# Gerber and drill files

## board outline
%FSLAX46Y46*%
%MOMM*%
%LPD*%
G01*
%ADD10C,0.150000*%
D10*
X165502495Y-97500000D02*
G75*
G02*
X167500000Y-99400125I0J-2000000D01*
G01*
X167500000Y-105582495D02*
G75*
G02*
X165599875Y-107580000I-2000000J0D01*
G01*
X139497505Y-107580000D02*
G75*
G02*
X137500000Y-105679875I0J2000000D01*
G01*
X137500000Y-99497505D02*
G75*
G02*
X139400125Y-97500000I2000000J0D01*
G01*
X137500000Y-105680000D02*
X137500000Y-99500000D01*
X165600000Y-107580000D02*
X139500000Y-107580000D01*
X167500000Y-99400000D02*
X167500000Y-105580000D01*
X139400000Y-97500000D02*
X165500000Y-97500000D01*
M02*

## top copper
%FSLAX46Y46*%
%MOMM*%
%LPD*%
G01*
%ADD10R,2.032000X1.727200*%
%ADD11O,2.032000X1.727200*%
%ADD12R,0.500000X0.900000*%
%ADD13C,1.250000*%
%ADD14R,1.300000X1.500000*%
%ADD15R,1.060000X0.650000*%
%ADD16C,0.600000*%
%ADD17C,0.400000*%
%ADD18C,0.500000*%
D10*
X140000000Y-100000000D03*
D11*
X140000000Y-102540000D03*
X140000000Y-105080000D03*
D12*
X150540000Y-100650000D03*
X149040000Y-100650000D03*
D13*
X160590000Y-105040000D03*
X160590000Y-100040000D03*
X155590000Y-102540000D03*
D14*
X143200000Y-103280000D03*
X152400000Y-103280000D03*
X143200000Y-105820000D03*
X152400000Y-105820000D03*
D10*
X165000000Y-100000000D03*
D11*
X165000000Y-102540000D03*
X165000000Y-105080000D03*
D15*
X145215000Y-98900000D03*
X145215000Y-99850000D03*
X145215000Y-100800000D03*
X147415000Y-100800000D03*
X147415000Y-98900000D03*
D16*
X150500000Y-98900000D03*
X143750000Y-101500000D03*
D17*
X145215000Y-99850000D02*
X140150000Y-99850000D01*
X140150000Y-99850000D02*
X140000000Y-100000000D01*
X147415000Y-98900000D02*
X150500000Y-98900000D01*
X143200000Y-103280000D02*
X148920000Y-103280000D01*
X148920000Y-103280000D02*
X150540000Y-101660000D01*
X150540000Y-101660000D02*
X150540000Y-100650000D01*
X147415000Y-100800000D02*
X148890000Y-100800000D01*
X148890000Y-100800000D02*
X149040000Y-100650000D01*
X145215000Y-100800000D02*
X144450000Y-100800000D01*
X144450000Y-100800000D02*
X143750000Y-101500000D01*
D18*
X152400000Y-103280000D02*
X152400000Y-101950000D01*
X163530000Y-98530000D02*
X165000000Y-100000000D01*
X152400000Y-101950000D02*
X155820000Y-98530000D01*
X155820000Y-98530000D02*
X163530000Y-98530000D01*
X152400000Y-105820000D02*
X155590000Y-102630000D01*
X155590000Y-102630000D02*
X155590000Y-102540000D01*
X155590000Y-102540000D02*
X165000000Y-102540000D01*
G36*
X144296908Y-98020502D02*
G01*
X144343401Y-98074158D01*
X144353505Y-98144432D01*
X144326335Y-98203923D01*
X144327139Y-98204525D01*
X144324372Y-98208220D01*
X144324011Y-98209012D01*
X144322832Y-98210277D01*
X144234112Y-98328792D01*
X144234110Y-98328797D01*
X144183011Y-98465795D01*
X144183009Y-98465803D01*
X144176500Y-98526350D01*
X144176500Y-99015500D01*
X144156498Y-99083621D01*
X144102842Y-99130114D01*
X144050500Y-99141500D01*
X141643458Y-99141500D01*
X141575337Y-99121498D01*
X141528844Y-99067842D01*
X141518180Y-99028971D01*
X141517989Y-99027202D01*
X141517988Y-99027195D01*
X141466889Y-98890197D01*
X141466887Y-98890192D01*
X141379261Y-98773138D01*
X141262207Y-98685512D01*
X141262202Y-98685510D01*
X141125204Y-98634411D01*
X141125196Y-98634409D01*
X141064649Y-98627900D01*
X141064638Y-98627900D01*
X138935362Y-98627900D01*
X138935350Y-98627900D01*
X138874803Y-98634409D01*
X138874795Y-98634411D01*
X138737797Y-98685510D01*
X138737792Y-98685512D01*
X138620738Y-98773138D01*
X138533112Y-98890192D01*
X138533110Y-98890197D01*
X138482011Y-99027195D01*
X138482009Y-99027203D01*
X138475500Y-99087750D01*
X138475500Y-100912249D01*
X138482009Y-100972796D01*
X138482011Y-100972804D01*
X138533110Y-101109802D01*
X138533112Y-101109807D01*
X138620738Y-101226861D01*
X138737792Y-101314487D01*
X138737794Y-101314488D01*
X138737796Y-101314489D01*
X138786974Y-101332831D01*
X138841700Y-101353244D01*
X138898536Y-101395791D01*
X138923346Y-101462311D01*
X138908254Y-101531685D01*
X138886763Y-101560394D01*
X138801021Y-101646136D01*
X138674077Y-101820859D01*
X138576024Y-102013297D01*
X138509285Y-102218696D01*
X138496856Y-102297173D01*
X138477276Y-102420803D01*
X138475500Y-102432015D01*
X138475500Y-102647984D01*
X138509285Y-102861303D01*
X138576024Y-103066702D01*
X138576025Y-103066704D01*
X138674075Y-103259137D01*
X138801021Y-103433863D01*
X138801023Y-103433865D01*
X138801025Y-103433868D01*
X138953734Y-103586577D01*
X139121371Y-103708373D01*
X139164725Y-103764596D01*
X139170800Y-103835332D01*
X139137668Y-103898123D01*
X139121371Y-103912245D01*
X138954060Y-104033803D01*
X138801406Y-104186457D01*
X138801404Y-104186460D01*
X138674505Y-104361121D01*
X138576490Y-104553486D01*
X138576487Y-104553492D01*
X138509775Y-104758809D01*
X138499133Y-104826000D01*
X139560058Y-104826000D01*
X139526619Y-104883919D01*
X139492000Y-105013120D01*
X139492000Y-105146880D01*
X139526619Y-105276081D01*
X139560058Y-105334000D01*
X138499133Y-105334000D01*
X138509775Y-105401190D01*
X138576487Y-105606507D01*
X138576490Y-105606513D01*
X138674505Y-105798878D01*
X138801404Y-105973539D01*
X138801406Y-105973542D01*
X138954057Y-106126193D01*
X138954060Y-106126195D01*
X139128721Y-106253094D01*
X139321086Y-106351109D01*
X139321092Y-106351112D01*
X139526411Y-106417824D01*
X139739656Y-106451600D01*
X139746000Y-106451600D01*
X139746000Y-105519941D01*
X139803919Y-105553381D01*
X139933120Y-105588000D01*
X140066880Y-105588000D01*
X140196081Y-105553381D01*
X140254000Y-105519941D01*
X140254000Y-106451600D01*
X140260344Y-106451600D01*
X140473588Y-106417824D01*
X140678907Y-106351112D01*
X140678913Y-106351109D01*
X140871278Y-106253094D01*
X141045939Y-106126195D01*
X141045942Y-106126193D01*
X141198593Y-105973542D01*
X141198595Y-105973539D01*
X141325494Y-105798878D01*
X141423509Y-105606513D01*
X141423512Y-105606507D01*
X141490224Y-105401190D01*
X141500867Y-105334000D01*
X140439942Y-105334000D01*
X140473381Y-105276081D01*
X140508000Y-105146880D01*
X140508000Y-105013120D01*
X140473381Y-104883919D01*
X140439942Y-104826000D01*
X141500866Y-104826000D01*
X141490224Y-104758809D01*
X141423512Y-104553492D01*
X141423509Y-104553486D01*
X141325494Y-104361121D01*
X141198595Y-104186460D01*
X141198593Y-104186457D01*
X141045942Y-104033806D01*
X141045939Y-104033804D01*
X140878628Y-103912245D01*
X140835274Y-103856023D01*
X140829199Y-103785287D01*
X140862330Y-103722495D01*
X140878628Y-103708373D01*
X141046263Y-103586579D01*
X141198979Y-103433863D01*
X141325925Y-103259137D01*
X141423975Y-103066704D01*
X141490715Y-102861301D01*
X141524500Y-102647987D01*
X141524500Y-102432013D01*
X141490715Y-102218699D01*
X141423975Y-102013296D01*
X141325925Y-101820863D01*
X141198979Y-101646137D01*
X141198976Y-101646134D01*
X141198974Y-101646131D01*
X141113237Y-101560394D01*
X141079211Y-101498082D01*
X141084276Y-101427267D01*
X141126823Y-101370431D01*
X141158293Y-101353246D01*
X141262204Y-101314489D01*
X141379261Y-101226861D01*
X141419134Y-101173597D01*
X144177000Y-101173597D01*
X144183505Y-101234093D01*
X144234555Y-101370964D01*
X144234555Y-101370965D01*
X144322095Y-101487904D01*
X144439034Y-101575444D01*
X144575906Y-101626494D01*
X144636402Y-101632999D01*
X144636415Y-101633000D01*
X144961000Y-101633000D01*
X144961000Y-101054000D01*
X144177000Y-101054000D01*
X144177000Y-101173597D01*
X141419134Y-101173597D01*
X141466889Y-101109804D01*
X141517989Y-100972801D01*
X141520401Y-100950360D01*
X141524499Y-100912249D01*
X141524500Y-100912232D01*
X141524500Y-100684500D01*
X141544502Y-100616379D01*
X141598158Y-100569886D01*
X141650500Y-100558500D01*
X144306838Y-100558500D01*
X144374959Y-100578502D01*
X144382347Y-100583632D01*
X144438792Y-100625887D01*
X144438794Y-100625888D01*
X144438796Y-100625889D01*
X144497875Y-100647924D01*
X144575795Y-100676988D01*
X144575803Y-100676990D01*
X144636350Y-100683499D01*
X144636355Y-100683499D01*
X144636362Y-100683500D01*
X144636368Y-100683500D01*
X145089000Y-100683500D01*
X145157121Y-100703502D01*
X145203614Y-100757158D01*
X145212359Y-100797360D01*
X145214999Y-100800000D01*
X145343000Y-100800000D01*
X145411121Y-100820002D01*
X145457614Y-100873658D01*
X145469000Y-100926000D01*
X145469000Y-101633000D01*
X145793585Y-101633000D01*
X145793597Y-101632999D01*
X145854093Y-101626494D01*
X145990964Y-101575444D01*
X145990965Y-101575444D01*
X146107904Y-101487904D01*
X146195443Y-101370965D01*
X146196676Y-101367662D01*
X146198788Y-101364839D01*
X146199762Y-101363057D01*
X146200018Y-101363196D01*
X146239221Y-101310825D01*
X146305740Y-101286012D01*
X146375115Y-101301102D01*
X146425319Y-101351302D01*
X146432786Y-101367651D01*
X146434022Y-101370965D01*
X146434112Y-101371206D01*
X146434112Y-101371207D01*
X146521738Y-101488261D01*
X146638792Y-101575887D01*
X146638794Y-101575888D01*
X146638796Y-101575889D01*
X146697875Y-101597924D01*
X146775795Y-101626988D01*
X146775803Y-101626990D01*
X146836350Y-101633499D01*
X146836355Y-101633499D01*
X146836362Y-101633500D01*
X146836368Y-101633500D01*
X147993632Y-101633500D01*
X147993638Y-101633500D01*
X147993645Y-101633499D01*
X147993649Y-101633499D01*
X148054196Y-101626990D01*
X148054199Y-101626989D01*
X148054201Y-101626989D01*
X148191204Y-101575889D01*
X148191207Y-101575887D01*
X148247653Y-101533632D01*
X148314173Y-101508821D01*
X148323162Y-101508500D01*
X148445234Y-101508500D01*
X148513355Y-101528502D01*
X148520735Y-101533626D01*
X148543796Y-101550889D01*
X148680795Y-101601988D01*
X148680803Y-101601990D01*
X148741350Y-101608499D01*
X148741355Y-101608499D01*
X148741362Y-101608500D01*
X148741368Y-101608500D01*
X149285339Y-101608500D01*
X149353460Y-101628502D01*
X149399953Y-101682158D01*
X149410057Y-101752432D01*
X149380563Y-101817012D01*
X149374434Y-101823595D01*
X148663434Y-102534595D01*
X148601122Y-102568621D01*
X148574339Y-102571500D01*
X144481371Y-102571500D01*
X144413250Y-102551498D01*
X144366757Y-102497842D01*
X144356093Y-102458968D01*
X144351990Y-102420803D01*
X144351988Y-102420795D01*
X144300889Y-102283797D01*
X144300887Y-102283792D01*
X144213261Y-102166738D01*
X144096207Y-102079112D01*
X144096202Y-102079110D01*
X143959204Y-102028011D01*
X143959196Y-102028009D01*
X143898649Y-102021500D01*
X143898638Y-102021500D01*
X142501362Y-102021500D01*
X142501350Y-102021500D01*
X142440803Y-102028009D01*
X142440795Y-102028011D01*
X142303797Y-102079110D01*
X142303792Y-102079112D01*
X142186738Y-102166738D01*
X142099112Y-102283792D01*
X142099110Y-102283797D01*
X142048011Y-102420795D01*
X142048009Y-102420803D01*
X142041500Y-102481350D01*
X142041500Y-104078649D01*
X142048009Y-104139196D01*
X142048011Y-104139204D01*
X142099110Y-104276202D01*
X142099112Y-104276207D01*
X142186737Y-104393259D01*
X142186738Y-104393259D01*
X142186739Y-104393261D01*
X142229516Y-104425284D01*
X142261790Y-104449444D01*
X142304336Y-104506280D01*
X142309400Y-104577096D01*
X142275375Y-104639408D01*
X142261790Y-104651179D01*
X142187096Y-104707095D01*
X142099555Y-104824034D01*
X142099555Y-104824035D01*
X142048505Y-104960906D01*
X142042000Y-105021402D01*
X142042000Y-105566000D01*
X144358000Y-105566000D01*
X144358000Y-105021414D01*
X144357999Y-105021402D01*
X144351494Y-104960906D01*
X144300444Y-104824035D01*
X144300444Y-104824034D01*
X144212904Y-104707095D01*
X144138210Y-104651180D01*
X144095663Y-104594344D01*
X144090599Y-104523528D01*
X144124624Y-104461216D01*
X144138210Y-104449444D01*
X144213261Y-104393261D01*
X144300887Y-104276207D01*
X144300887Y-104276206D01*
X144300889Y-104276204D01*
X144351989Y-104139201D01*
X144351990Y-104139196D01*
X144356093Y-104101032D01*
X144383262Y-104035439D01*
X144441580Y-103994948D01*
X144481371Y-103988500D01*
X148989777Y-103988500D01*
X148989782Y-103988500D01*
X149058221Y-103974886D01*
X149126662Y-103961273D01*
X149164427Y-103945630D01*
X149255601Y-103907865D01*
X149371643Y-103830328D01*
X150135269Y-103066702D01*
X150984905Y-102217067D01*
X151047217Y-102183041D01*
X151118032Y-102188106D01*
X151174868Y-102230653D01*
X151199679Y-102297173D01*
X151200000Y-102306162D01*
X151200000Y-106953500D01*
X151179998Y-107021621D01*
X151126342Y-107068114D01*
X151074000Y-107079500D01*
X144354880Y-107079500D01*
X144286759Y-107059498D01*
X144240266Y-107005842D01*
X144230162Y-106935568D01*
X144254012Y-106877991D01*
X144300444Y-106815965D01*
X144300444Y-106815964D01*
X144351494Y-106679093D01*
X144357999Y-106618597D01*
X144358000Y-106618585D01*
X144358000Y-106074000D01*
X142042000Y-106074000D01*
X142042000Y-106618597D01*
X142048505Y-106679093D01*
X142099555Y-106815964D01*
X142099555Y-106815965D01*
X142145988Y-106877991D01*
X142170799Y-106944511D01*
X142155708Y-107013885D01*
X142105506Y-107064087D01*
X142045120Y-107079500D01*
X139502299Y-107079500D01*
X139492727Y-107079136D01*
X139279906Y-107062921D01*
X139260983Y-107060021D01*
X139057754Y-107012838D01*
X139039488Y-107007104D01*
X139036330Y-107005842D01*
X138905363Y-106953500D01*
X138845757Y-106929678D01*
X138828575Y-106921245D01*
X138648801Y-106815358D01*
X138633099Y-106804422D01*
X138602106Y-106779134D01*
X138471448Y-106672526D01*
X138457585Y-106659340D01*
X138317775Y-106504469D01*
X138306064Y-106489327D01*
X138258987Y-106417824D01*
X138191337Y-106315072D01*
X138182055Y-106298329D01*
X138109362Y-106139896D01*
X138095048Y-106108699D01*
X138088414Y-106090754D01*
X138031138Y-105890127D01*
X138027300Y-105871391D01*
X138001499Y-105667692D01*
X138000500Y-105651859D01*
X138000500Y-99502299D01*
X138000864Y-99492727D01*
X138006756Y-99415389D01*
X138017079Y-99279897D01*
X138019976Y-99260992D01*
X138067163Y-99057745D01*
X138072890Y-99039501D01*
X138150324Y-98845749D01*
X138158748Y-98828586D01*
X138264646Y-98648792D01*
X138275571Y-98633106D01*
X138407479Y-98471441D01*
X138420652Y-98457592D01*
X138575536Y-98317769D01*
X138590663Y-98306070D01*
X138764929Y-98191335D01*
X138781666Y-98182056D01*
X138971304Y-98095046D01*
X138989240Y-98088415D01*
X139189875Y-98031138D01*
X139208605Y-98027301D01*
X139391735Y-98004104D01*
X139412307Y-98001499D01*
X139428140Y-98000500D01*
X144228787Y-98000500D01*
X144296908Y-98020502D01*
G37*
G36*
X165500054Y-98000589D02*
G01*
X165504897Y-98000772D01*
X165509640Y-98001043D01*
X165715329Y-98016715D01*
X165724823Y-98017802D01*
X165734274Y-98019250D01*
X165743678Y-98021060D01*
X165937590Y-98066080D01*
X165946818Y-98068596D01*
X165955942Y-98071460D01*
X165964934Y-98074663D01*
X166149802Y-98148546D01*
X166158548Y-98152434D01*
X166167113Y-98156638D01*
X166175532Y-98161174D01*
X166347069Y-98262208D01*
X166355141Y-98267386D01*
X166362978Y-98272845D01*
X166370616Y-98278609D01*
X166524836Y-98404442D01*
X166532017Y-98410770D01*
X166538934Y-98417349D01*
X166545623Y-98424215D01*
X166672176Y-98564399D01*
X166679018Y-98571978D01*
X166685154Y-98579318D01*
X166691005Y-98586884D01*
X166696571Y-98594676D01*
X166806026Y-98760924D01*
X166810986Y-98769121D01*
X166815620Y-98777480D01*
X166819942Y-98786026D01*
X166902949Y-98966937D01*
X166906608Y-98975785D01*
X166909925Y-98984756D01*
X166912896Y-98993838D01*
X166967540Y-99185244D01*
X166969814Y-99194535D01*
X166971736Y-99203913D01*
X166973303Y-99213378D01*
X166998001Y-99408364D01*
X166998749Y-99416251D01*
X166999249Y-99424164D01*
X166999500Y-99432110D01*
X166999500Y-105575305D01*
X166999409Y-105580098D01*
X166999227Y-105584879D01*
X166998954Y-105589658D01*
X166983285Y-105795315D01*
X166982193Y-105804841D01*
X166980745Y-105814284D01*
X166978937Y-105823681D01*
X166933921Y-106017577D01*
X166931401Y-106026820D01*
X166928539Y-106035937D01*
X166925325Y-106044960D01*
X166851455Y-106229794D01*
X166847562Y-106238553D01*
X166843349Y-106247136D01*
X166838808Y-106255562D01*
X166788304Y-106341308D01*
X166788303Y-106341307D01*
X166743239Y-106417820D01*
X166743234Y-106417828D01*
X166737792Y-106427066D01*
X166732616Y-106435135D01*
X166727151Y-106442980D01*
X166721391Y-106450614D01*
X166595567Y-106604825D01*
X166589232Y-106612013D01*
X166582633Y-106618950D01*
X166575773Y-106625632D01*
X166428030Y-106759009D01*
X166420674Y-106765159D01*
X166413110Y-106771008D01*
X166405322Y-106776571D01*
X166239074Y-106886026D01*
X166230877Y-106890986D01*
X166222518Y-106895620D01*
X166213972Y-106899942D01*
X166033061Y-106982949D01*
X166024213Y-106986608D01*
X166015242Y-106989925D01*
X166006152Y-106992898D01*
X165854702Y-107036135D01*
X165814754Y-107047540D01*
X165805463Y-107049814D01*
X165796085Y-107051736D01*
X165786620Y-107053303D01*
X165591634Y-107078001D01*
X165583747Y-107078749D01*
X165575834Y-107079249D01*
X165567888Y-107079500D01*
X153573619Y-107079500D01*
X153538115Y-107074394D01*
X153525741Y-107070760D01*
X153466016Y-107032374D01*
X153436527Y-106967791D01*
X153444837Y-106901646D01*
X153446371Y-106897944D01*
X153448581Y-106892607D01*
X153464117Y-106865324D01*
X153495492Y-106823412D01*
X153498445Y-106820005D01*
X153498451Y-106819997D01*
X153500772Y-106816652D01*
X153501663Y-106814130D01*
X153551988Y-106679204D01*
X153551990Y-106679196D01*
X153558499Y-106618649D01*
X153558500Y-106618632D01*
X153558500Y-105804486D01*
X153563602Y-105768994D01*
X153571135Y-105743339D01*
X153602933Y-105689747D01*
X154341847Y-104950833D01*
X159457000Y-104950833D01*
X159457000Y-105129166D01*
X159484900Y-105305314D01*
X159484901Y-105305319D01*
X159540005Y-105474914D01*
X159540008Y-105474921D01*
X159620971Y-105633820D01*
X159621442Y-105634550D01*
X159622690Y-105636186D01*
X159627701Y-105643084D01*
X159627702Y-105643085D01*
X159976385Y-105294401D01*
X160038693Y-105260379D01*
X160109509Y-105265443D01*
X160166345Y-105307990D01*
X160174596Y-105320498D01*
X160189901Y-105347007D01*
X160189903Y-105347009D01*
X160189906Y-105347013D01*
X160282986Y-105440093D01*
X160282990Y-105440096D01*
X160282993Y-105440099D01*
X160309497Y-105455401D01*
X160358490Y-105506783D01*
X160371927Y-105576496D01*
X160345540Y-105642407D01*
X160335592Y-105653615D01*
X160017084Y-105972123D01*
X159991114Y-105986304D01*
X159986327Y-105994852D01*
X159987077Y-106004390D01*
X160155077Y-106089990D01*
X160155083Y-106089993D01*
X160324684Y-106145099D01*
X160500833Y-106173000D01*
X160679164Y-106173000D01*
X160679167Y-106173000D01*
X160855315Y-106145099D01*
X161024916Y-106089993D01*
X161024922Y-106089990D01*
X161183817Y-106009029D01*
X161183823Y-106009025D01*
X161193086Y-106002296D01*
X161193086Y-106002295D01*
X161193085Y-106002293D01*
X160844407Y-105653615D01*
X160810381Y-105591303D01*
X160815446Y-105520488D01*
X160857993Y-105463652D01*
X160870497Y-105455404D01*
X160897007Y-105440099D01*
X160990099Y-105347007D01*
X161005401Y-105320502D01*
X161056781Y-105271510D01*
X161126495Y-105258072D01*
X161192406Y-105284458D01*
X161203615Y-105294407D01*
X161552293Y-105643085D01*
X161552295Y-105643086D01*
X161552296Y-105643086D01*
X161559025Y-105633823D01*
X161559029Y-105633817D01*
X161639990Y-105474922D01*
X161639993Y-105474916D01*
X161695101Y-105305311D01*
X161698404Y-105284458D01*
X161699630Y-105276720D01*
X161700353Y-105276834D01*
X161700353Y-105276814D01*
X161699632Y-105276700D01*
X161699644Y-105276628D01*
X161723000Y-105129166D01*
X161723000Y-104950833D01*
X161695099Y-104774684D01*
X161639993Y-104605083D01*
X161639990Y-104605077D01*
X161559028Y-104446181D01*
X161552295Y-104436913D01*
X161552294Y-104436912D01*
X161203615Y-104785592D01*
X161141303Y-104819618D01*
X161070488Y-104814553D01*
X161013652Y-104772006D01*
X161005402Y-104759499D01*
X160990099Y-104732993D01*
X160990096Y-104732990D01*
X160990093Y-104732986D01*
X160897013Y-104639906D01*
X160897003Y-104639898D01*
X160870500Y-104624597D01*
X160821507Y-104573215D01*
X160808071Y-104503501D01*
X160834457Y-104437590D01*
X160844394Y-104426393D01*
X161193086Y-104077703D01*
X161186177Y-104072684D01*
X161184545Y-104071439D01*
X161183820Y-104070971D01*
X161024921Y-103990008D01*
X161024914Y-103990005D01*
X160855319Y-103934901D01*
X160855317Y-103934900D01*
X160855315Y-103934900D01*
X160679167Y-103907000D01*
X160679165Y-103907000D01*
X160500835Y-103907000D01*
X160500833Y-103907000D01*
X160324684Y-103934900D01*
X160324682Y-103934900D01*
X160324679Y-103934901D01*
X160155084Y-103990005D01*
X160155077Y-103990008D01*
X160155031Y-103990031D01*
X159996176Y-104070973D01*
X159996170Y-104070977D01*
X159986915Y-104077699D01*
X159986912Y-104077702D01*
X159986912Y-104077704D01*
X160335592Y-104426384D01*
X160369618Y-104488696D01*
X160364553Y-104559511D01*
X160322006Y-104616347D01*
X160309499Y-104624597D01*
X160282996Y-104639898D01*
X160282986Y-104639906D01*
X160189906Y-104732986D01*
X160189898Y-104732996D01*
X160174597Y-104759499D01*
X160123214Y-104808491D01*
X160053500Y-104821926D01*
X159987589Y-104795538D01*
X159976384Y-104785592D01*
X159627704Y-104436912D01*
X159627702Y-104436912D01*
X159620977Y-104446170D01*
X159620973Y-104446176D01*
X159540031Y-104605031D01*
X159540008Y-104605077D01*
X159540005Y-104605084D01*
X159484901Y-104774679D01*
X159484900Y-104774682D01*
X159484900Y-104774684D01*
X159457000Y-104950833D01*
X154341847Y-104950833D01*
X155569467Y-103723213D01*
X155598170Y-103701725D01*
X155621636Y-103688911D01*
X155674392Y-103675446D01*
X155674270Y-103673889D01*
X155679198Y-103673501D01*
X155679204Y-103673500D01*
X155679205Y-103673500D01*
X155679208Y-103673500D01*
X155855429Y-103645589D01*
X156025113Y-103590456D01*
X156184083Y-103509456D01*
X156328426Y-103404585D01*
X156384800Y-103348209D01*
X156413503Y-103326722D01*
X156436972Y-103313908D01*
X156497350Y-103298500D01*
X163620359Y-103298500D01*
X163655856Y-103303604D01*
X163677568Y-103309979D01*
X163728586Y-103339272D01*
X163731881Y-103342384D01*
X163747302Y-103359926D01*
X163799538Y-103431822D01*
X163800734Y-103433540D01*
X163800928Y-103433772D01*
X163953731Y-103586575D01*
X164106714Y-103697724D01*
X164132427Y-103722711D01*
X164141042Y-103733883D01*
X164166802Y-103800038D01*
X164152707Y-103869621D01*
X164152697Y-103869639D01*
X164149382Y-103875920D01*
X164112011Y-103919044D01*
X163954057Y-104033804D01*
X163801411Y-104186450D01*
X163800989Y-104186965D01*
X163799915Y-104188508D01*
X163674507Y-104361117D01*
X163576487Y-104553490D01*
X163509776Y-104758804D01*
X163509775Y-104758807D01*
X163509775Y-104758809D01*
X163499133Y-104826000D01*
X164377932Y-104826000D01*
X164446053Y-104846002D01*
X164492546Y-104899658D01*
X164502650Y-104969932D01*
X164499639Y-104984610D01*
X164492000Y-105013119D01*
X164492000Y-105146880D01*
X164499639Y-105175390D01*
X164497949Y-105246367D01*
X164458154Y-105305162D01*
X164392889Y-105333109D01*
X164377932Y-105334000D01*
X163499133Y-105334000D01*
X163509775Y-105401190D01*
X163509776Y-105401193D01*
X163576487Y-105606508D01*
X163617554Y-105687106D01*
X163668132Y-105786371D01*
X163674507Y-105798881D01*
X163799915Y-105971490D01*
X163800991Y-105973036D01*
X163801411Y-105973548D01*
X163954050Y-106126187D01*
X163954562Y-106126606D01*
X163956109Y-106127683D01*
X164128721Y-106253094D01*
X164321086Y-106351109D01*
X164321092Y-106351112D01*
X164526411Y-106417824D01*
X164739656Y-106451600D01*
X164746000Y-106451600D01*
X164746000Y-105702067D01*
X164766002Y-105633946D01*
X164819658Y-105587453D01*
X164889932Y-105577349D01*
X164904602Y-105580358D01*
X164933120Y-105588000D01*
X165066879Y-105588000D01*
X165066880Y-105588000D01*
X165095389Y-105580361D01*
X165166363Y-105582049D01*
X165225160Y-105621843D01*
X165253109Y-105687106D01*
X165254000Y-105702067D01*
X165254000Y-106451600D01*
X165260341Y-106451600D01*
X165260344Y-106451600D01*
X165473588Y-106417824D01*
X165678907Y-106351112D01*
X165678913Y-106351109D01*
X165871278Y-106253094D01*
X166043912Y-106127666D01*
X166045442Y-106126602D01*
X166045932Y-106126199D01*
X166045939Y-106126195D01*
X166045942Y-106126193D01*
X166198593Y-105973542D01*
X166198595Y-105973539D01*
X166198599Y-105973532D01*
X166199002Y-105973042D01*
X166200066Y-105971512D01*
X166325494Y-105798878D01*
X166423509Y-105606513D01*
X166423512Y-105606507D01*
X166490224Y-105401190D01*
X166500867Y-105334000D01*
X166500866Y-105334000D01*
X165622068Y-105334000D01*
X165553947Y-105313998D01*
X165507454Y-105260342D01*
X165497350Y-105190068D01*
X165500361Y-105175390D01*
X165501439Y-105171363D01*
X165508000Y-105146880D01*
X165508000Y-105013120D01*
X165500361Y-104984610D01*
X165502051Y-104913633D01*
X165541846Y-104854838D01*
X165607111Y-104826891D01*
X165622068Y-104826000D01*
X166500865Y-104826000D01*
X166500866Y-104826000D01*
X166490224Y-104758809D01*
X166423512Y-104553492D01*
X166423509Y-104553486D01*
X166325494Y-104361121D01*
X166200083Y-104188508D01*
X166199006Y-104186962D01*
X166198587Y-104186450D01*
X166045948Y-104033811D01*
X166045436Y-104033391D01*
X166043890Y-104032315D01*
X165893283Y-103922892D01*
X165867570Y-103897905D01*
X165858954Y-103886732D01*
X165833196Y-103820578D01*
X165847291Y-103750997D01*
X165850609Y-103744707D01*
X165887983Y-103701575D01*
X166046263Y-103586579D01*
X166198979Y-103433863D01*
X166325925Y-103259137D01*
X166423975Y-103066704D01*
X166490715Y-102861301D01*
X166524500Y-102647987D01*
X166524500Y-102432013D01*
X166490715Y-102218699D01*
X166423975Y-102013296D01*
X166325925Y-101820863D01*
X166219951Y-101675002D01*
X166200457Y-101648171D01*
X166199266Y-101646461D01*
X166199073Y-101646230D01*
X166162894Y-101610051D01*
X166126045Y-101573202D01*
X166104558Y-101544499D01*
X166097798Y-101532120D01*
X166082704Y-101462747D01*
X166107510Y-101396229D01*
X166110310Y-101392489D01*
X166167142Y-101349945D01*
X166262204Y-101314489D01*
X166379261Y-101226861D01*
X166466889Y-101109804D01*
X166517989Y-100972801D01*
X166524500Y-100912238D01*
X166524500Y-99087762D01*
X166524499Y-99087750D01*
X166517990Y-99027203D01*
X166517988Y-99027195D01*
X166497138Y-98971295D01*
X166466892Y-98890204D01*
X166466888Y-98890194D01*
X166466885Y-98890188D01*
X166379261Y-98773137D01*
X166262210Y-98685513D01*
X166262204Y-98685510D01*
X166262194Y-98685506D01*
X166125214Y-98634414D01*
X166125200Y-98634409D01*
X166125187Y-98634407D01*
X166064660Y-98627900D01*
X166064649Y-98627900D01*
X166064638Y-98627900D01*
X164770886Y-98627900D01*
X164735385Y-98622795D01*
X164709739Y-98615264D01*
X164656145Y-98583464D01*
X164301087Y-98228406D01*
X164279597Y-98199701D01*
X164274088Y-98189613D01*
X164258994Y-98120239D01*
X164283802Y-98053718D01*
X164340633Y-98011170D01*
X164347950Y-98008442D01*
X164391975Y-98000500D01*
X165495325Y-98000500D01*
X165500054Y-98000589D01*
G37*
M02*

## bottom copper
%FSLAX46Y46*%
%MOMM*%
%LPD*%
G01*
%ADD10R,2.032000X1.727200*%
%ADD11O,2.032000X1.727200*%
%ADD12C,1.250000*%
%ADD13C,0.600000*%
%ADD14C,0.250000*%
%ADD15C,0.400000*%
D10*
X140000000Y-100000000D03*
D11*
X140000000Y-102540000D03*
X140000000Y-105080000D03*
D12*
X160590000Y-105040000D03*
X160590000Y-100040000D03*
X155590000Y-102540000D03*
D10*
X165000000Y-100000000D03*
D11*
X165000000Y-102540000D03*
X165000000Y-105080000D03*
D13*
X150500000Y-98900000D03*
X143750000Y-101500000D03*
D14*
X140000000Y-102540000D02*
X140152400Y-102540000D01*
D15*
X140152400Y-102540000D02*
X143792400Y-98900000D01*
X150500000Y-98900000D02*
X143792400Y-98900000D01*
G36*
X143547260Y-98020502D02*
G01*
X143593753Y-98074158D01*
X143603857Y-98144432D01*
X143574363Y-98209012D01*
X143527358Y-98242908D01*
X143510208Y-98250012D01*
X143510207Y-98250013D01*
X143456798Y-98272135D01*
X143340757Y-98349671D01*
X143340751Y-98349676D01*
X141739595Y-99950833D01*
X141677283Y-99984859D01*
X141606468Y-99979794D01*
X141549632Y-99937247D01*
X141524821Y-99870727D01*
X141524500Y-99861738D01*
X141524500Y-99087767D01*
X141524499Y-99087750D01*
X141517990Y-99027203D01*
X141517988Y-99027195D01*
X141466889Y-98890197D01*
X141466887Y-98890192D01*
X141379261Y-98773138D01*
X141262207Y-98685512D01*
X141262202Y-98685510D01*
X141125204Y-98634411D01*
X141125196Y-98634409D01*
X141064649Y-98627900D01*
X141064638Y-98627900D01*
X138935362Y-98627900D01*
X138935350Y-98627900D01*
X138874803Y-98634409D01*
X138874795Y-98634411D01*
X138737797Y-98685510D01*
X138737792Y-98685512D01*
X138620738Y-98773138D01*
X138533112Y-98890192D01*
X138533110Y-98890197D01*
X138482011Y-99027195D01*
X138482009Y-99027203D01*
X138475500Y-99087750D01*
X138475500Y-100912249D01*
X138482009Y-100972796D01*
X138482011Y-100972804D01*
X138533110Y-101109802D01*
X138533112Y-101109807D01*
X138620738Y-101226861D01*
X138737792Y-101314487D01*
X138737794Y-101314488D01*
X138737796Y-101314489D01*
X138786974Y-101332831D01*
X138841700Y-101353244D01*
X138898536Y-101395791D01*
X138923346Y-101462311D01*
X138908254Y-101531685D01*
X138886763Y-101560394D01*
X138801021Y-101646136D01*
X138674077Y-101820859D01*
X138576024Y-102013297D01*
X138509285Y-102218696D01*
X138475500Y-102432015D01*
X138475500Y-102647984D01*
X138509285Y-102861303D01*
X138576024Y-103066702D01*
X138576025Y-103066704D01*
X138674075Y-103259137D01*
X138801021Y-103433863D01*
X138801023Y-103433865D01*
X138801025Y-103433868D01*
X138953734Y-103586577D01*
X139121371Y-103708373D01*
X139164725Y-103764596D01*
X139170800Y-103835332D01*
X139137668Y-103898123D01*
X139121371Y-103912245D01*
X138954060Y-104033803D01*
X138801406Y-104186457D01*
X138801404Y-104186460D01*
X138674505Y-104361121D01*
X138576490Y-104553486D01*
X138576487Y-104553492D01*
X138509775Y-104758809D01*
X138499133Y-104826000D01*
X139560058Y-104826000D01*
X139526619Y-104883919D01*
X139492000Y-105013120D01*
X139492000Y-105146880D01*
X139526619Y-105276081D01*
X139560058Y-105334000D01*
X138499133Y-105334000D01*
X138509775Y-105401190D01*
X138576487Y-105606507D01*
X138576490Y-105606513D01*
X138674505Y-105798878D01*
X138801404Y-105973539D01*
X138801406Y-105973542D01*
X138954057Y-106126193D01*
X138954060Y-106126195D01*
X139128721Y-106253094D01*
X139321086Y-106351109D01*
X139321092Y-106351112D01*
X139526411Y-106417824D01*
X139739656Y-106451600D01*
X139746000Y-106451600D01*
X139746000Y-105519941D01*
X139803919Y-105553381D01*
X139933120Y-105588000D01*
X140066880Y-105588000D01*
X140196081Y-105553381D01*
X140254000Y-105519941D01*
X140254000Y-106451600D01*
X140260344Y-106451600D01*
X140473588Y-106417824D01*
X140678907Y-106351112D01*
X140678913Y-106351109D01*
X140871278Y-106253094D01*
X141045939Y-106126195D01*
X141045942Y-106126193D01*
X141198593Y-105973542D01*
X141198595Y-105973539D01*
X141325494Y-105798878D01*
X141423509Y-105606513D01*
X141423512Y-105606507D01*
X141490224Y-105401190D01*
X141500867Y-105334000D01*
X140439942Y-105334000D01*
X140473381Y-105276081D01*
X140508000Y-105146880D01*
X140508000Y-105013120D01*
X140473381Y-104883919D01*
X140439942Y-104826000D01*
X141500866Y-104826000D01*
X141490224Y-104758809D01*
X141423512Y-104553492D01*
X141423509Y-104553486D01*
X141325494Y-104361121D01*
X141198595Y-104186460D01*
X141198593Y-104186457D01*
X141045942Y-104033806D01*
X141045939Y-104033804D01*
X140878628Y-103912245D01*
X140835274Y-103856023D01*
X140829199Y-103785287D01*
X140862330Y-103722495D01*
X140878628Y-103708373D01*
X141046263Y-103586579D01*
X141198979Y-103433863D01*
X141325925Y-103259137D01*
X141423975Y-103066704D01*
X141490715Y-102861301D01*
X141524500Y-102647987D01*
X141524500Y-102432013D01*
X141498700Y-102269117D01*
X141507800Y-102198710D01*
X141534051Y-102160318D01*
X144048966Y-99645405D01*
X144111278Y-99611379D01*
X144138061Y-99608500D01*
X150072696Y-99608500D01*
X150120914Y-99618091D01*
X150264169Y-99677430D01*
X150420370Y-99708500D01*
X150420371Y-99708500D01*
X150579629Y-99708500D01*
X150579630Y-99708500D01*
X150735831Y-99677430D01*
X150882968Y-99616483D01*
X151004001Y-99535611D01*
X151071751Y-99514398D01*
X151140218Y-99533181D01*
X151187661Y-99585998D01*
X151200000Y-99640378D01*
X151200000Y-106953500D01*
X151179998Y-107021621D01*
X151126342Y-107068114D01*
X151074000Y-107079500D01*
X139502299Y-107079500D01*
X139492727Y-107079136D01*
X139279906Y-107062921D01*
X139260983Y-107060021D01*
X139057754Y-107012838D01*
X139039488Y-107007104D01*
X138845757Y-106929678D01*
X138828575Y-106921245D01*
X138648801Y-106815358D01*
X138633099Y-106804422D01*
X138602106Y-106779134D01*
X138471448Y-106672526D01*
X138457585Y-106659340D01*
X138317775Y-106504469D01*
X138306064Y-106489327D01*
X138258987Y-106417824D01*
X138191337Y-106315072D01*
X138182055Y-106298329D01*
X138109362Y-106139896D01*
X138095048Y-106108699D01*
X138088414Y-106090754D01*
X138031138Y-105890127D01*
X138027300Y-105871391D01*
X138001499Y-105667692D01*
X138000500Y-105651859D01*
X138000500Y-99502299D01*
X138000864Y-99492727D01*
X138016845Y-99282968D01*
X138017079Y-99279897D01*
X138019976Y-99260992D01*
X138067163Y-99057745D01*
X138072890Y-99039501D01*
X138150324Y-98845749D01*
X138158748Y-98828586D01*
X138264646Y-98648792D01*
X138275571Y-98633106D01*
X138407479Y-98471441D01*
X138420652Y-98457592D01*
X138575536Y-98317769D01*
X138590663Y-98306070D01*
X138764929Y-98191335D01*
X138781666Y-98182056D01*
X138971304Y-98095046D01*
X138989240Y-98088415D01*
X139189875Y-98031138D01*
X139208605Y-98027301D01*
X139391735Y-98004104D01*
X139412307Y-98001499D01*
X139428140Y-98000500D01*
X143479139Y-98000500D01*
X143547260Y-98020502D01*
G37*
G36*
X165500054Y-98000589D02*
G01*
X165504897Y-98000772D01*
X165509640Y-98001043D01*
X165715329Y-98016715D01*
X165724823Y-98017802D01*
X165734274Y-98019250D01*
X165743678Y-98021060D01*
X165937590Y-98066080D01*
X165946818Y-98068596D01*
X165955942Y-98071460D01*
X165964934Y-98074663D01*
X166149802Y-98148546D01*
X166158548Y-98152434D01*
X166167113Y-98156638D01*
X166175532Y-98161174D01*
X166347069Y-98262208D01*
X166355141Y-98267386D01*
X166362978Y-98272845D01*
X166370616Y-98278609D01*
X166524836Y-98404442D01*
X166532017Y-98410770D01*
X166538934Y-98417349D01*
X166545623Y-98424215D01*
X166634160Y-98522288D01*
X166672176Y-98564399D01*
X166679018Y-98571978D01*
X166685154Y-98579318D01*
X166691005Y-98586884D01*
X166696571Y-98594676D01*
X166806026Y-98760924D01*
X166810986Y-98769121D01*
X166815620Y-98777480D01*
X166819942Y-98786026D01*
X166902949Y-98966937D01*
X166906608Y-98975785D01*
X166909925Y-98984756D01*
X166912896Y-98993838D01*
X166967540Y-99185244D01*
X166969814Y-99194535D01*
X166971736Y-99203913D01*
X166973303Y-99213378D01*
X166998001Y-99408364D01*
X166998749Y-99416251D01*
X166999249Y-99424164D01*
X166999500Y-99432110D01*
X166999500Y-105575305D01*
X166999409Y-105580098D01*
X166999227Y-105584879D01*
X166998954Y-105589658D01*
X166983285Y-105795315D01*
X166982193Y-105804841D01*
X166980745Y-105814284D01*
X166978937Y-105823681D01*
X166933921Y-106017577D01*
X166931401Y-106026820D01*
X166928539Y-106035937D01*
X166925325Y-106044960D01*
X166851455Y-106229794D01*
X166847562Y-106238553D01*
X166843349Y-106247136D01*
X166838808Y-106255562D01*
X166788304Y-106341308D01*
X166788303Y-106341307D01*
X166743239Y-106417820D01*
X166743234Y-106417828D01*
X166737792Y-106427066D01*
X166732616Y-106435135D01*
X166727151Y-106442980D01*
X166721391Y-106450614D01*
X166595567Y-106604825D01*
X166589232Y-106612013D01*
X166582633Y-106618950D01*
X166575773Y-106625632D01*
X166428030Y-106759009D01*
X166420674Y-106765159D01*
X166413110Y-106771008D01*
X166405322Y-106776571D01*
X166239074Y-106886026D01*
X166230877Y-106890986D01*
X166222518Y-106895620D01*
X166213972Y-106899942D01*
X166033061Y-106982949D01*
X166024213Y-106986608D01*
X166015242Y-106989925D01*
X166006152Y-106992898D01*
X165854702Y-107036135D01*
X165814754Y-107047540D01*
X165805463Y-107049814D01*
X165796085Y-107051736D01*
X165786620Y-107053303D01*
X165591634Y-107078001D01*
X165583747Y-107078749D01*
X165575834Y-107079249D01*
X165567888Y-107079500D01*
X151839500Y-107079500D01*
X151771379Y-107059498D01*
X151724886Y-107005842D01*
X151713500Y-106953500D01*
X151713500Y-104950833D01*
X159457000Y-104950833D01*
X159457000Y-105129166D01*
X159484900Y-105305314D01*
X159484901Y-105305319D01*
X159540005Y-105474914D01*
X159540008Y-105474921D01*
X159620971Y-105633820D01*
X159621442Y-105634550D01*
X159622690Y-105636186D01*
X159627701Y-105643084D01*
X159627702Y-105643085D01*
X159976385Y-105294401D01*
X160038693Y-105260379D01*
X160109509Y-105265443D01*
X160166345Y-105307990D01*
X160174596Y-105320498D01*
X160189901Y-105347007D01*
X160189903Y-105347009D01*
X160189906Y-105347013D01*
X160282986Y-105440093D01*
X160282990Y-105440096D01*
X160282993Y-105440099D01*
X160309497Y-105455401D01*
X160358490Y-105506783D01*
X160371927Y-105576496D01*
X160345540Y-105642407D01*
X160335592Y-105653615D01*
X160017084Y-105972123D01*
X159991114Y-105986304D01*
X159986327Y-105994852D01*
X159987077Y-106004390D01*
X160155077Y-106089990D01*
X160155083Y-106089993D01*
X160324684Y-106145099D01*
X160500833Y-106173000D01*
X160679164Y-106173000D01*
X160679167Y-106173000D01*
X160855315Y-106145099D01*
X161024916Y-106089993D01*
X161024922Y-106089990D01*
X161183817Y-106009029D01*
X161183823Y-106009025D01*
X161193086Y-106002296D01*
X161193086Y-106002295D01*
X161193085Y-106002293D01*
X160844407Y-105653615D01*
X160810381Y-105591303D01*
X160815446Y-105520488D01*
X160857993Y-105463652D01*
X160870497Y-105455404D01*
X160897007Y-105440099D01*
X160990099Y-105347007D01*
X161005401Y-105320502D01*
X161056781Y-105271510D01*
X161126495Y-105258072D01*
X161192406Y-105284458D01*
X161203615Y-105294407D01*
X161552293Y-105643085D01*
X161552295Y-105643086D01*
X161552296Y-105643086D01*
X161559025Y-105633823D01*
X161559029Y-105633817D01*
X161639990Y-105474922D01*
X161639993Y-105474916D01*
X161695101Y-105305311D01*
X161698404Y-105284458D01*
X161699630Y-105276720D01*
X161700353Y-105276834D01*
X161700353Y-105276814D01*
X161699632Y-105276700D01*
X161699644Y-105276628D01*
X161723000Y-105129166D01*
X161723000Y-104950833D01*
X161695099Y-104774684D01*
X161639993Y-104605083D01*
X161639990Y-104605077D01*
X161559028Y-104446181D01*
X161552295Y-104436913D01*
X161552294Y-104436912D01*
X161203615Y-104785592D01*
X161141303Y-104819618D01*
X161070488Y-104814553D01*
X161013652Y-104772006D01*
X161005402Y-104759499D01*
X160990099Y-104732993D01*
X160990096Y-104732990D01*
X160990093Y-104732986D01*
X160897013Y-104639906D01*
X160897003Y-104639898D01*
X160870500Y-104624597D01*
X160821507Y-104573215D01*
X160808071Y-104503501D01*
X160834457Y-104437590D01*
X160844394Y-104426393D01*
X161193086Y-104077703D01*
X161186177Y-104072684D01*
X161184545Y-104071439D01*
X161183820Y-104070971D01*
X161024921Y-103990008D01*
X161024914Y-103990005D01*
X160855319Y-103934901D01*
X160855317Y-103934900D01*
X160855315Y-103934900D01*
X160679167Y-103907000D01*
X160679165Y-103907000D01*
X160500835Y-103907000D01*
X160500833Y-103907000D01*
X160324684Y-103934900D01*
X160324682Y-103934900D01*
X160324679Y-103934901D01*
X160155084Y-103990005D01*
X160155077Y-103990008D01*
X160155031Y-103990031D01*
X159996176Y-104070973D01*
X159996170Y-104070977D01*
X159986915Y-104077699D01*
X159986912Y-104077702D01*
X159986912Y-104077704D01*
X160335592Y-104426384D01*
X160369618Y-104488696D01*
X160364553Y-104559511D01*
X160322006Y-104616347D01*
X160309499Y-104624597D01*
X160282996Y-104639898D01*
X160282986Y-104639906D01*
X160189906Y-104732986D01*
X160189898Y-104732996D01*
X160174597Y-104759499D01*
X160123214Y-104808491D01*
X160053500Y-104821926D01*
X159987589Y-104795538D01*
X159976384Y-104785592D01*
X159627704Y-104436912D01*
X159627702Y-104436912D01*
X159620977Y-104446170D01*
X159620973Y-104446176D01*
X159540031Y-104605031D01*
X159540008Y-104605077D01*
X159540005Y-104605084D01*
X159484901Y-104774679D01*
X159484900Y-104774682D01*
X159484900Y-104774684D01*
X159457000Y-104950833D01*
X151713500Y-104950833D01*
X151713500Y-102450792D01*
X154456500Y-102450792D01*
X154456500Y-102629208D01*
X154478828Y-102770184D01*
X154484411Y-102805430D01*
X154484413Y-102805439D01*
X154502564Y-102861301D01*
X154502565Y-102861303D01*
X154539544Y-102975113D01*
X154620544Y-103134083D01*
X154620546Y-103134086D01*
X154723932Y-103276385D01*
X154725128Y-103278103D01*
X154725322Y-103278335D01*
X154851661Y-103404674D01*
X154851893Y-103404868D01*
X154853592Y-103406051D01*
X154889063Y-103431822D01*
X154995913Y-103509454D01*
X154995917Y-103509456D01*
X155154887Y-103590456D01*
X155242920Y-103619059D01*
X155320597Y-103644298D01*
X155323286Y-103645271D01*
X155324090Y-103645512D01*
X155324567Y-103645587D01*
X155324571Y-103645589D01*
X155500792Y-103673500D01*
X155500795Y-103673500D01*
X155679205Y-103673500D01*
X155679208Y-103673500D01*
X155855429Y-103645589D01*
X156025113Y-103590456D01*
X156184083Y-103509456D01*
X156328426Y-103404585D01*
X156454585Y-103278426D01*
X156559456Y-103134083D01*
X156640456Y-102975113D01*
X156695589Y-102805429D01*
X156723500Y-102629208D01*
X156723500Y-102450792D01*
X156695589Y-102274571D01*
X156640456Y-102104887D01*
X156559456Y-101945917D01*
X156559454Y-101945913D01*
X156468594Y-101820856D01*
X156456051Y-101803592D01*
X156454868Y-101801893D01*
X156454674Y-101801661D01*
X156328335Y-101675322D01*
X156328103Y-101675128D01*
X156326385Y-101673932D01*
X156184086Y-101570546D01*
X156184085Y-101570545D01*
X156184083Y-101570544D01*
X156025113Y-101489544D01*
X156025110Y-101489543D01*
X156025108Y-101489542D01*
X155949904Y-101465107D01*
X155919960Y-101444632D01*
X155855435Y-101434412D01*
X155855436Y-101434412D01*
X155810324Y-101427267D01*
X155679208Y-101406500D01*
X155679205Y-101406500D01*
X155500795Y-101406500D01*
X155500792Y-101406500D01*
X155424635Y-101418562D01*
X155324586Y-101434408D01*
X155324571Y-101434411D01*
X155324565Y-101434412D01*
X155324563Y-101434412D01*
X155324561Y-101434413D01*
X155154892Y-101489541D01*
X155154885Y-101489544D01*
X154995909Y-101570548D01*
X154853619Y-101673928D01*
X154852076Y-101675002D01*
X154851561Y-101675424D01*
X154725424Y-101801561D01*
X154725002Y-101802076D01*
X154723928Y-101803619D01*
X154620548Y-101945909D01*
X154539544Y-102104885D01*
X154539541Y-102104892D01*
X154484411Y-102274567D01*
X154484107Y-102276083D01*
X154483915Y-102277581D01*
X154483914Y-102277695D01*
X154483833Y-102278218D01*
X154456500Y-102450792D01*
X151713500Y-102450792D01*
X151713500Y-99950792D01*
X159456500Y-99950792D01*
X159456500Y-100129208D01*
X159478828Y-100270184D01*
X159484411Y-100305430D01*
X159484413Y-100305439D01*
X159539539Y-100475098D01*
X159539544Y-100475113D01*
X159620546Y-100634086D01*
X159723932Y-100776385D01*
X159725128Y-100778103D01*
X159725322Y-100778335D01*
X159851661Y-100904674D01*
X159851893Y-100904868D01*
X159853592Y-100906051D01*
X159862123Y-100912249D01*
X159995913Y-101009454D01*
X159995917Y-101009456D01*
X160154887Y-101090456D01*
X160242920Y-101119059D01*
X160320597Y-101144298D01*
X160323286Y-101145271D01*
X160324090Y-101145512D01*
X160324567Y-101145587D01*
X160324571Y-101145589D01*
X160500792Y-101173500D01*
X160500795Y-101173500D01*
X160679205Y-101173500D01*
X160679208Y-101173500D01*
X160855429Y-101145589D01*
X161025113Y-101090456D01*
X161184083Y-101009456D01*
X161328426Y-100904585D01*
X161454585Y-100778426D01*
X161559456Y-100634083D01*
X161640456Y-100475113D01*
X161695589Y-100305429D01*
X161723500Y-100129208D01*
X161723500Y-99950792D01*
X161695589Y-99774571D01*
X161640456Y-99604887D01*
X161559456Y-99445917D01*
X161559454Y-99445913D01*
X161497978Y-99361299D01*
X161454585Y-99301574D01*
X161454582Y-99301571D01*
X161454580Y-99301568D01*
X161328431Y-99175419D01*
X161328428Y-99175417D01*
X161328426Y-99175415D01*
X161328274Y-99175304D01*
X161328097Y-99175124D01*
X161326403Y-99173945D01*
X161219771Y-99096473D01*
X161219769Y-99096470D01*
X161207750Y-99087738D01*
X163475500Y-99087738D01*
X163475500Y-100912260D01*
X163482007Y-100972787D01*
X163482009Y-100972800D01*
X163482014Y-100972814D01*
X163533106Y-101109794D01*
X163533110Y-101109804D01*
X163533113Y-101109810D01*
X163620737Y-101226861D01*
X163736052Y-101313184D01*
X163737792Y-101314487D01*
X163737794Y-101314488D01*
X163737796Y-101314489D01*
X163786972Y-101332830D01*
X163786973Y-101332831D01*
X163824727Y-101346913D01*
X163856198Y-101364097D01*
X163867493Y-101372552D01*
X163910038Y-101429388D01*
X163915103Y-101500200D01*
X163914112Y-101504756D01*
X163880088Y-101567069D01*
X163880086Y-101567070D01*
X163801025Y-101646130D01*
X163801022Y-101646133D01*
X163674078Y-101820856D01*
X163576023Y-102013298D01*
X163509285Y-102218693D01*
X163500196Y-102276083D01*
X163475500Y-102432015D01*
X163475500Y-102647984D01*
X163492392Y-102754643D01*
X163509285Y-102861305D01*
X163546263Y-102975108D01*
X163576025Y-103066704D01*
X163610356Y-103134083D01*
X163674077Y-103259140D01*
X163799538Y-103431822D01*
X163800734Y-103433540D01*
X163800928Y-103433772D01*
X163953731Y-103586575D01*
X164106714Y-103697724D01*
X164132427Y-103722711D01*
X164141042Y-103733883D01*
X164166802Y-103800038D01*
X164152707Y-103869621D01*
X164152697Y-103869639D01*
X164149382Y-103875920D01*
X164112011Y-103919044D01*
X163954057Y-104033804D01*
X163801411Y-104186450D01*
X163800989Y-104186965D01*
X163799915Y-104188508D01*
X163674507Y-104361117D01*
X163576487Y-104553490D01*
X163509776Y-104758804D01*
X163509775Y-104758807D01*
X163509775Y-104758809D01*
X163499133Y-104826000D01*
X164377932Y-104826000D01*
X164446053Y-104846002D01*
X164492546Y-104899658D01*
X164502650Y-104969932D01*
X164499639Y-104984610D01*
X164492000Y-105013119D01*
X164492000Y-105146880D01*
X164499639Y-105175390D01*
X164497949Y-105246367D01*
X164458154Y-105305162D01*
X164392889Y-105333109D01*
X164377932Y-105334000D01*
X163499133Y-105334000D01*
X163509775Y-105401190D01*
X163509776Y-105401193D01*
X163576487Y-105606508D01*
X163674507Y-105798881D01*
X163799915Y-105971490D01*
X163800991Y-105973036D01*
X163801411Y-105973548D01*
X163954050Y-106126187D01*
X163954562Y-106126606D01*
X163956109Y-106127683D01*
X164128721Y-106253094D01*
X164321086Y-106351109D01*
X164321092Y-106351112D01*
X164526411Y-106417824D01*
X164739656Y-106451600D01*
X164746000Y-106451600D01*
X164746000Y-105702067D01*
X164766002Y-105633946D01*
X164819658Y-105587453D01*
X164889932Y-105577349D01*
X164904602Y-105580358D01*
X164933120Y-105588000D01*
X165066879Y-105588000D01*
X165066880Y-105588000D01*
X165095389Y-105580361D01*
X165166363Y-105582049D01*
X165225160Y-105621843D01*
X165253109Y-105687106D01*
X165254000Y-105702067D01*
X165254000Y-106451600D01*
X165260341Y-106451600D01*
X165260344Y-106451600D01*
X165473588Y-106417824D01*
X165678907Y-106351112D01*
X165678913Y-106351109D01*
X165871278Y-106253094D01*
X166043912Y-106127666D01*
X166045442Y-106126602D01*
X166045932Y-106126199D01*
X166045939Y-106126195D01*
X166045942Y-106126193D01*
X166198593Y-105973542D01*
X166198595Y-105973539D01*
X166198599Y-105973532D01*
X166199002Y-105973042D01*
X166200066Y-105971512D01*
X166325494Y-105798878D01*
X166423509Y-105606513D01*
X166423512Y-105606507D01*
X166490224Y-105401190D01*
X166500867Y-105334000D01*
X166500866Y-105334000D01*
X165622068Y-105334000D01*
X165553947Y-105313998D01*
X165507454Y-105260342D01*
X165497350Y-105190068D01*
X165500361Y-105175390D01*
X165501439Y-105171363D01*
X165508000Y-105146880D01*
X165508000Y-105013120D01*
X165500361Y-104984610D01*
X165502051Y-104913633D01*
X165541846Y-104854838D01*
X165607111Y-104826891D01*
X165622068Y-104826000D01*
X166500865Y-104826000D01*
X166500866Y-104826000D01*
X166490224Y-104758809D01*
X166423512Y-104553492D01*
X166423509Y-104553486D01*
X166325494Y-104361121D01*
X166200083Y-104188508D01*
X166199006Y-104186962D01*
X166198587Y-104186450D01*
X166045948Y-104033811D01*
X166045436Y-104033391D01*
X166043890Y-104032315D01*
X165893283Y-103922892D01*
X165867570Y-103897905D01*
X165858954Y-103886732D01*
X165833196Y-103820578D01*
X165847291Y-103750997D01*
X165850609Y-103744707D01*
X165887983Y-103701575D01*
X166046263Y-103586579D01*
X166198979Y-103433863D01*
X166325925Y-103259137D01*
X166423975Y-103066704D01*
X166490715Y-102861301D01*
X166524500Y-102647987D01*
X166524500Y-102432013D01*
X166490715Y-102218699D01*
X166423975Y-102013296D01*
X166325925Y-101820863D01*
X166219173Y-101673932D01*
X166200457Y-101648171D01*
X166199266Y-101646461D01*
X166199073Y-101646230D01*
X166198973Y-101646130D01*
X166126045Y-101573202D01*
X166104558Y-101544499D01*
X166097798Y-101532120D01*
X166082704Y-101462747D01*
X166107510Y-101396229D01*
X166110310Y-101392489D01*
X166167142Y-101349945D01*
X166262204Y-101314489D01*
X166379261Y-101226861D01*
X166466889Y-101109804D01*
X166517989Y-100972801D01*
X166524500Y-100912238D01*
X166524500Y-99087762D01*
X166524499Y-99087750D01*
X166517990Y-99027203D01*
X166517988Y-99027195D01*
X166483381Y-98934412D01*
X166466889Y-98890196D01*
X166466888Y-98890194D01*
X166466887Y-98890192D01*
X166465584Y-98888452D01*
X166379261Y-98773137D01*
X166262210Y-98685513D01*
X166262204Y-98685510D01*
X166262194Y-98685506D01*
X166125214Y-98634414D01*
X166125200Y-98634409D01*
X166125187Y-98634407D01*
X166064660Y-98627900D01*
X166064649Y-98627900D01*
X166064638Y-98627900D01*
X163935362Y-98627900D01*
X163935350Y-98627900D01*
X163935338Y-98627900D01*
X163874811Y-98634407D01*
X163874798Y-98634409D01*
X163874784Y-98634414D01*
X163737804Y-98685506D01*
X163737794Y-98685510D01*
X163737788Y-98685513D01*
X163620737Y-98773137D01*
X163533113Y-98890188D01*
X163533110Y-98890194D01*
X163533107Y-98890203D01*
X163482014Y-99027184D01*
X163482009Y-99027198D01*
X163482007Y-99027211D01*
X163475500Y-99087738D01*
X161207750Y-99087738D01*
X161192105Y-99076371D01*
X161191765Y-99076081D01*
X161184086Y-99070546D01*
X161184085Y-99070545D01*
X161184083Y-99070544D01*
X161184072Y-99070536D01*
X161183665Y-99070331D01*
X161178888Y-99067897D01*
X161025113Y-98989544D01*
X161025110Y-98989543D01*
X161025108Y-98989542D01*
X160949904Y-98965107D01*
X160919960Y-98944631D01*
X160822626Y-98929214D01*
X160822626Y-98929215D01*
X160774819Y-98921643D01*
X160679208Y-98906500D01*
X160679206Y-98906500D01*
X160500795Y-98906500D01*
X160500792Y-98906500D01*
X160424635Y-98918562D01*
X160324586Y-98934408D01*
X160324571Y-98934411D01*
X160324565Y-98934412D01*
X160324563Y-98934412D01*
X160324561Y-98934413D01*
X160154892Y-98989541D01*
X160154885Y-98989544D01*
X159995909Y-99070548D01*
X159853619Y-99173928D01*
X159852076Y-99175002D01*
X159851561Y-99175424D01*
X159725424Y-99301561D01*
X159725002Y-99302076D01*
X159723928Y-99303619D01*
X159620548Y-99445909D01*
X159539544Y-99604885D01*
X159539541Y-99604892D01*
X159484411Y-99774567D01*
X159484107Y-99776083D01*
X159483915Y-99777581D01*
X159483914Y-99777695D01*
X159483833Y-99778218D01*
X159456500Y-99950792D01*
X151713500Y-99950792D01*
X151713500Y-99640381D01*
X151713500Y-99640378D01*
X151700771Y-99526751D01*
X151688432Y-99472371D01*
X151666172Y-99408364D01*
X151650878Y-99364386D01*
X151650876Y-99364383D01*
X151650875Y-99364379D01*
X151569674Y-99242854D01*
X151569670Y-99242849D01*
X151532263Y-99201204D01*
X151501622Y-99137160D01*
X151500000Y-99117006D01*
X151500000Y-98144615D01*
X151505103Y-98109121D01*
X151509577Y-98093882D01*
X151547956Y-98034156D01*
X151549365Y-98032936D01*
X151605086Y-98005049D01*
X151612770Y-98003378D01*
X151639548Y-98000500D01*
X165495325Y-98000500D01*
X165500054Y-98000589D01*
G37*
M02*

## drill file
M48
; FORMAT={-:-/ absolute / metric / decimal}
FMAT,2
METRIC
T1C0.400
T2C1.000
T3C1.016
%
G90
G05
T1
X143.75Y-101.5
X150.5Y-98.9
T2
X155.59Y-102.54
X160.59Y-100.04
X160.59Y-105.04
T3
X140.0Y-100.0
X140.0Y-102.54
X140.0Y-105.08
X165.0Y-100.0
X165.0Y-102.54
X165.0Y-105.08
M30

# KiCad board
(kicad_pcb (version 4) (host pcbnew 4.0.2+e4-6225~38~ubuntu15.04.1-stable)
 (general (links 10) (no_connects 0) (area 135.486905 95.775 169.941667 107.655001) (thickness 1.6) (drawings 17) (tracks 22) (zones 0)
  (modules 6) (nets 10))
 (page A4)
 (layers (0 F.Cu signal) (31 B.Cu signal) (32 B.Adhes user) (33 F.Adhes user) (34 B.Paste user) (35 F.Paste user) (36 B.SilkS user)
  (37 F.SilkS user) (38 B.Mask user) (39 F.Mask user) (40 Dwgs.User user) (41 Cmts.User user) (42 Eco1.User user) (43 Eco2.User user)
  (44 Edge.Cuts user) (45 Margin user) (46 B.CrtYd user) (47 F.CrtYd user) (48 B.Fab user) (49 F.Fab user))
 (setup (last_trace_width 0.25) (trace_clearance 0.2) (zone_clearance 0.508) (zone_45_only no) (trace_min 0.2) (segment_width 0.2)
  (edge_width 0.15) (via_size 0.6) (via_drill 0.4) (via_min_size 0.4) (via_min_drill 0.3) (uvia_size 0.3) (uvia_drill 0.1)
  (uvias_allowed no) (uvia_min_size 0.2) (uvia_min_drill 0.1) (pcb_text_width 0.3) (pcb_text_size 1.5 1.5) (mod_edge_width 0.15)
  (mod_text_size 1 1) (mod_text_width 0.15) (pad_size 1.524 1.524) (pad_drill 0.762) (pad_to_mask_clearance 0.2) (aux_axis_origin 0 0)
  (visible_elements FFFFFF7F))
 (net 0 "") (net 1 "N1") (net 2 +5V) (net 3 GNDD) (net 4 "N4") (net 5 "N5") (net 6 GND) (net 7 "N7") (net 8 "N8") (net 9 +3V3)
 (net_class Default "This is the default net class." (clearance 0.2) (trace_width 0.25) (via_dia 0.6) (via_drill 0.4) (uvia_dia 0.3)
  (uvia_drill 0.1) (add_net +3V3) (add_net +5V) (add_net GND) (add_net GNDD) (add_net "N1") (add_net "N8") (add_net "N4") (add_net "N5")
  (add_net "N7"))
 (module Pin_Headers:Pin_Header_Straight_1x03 (layer F.Cu) (at 140 100)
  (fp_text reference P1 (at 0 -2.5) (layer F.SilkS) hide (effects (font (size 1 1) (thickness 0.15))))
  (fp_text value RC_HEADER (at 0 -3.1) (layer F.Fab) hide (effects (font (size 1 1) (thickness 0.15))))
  (pad 1 thru_hole rect (at 0 0) (size 2.032 1.7272) (drill 1.016) (layers *.Cu *.Mask F.SilkS) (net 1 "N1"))
  (pad 2 thru_hole oval (at 0 2.54) (size 2.032 1.7272) (drill 1.016) (layers *.Cu *.Mask F.SilkS) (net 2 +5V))
  (pad 3 thru_hole oval (at 0 5.08) (size 2.032 1.7272) (drill 1.016) (layers *.Cu *.Mask F.SilkS) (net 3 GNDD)))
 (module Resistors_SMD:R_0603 (layer F.Cu) (at 149.79 100.65 180)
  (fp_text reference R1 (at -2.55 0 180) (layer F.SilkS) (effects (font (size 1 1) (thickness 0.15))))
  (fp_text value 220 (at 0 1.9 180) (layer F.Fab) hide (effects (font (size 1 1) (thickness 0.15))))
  (pad 1 smd rect (at -0.75 0 180) (size 0.5 0.9) (layers F.Cu F.Paste F.Mask) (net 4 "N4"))
  (pad 2 smd rect (at 0.75 0 180) (size 0.5 0.9) (layers F.Cu F.Paste F.Mask) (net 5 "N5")))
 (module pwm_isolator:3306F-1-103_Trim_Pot (layer F.Cu) (at 160.59 102.54 90)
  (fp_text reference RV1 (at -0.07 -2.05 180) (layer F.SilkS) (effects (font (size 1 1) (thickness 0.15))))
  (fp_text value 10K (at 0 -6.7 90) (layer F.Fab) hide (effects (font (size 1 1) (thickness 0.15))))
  (pad 1 thru_hole circle (at -2.5 0 90) (size 1.25 1.25) (drill 1) (layers *.Cu *.Mask) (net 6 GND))
  (pad 3 thru_hole circle (at 2.5 0 90) (size 1.25 1.25) (drill 1) (layers *.Cu *.Mask) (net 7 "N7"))
  (pad 2 thru_hole circle (at 0 -5 90) (size 1.25 1.25) (drill 1) (layers *.Cu *.Mask) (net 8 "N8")))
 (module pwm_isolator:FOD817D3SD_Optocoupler (layer F.Cu) (at 147.8 104.55)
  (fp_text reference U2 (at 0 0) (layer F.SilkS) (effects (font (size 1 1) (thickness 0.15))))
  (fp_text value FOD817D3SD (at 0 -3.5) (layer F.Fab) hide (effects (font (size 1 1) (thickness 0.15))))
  (pad 1 smd rect (at -4.6 -1.27) (size 1.3 1.5) (layers F.Cu F.Paste F.Mask) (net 4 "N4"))
  (pad 4 smd rect (at 4.6 -1.27) (size 1.3 1.5) (layers F.Cu F.Paste F.Mask) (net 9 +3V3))
  (pad 2 smd rect (at -4.6 1.27) (size 1.3 1.5) (layers F.Cu F.Paste F.Mask) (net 3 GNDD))
  (pad 3 smd rect (at 4.6 1.27) (size 1.3 1.5) (layers F.Cu F.Paste F.Mask) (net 8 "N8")))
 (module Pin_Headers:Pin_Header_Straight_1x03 (layer F.Cu) (at 165 100)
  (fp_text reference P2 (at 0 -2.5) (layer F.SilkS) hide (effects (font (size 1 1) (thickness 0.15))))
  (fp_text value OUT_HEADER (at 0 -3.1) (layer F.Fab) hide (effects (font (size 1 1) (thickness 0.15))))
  (pad 1 thru_hole rect (at 0 0) (size 2.032 1.7272) (drill 1.016) (layers *.Cu *.Mask F.SilkS) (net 9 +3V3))
  (pad 2 thru_hole oval (at 0 2.54) (size 2.032 1.7272) (drill 1.016) (layers *.Cu *.Mask F.SilkS) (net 8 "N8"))
  (pad 3 thru_hole oval (at 0 5.08) (size 2.032 1.7272) (drill 1.016) (layers *.Cu *.Mask F.SilkS) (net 6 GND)))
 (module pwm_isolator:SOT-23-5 (layer F.Cu) (at 146.315 99.85)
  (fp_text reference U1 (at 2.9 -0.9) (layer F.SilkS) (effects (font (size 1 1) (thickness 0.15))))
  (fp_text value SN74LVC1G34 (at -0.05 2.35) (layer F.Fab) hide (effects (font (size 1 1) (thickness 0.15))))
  (pad 1 smd rect (at -1.1 -0.95) (size 1.06 0.65) (layers F.Cu F.Paste F.Mask))
  (pad 2 smd rect (at -1.1 0) (size 1.06 0.65) (layers F.Cu F.Paste F.Mask) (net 1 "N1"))
  (pad 3 smd rect (at -1.1 0.95) (size 1.06 0.65) (layers F.Cu F.Paste F.Mask) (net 3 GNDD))
  (pad 4 smd rect (at 1.1 0.95) (size 1.06 0.65) (layers F.Cu F.Paste F.Mask) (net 5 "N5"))
  (pad 5 smd rect (at 1.1 -0.95) (size 1.06 0.65) (layers F.Cu F.Paste F.Mask) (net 2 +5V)))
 (gr_arc (start 165.502495 99.5) (end 165.502495 97.5) (angle 87.13759477) (layer Edge.Cuts) (width 0.15))
 (gr_arc (start 165.5 105.582495) (end 167.5 105.582495) (angle 87.13759477) (layer Edge.Cuts) (width 0.15))
 (gr_arc (start 139.497505 105.58) (end 139.497505 107.58) (angle 87.13759477) (layer Edge.Cuts) (width 0.15))
 (gr_arc (start 139.5 99.497505) (end 137.5 99.497505) (angle 87.13759477) (layer Edge.Cuts) (width 0.15))
 (gr_line (start 137.5 105.68) (end 137.5 99.5) (layer Edge.Cuts) (width 0.15))
 (gr_line (start 165.6 107.58) (end 139.5 107.58) (layer Edge.Cuts) (width 0.15))
 (gr_line (start 167.5 99.4) (end 167.5 105.58) (layer Edge.Cuts) (width 0.15))
 (gr_line (start 139.4 97.5) (end 165.5 97.5) (layer Edge.Cuts) (width 0.15))
 (segment (start 145.215 99.85) (end 140.15 99.85) (width 0.4) (layer F.Cu) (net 1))
 (segment (start 140.15 99.85) (end 140 100) (width 0.4) (layer F.Cu) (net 1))
 (segment (start 140 102.54) (end 140.1524 102.54) (width 0.25) (layer B.Cu) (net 2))
 (segment (start 140.1524 102.54) (end 143.7924 98.9) (width 0.4) (layer B.Cu) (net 2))
 (segment (start 150.5 98.9) (end 143.7924 98.9) (width 0.4) (layer B.Cu) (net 2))
 (segment (start 147.415 98.9) (end 150.5 98.9) (width 0.4) (layer F.Cu) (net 2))
 (via (at 150.5 98.9) (size 0.6) (drill 0.4) (layers F.Cu B.Cu) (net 2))
 (segment (start 143.2 103.28) (end 148.92 103.28) (width 0.4) (layer F.Cu) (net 4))
 (segment (start 148.92 103.28) (end 150.54 101.66) (width 0.4) (layer F.Cu) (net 4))
 (segment (start 150.54 101.66) (end 150.54 100.65) (width 0.4) (layer F.Cu) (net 4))
 (segment (start 147.415 100.8) (end 148.89 100.8) (width 0.4) (layer F.Cu) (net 5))
 (segment (start 148.89 100.8) (end 149.04 100.65) (width 0.4) (layer F.Cu) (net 5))
 (segment (start 145.215 100.8) (end 144.45 100.8) (width 0.4) (layer F.Cu) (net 3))
 (segment (start 144.45 100.8) (end 143.75 101.5) (width 0.4) (layer F.Cu) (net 3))
 (via (at 143.75 101.5) (size 0.6) (drill 0.4) (layers F.Cu B.Cu) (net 3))
 (segment (start 152.4 103.28) (end 152.4 101.95) (width 0.5) (layer F.Cu) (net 9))
 (segment (start 163.53 98.53) (end 165 100) (width 0.5) (layer F.Cu) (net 9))
 (segment (start 152.4 101.95) (end 155.82 98.53) (width 0.5) (layer F.Cu) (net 9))
 (segment (start 155.82 98.53) (end 163.53 98.53) (width 0.5) (layer F.Cu) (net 9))
 (segment (start 152.4 105.82) (end 155.59 102.63) (width 0.5) (layer F.Cu) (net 8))
 (segment (start 155.59 102.63) (end 155.59 102.54) (width 0.5) (layer F.Cu) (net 8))
 (segment (start 155.59 102.54) (end 165 102.54) (width 0.5) (layer F.Cu) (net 8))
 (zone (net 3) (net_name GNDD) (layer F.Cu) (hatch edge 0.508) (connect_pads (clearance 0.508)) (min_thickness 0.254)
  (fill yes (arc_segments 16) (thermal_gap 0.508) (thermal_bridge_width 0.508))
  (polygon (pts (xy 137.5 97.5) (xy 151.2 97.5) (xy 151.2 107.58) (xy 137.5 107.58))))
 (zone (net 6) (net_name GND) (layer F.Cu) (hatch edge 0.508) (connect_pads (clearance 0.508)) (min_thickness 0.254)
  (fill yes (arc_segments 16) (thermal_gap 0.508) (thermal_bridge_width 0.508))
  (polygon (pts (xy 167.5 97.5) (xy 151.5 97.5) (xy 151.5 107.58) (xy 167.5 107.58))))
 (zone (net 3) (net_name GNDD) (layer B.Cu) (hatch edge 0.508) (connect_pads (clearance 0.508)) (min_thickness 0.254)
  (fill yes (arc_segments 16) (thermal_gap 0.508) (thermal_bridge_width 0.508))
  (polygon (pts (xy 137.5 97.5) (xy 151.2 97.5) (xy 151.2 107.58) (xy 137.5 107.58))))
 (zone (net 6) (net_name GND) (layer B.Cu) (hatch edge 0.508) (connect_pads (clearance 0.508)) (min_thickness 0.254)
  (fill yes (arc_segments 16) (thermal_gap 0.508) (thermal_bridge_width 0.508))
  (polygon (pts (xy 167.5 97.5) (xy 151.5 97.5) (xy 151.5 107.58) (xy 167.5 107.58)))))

